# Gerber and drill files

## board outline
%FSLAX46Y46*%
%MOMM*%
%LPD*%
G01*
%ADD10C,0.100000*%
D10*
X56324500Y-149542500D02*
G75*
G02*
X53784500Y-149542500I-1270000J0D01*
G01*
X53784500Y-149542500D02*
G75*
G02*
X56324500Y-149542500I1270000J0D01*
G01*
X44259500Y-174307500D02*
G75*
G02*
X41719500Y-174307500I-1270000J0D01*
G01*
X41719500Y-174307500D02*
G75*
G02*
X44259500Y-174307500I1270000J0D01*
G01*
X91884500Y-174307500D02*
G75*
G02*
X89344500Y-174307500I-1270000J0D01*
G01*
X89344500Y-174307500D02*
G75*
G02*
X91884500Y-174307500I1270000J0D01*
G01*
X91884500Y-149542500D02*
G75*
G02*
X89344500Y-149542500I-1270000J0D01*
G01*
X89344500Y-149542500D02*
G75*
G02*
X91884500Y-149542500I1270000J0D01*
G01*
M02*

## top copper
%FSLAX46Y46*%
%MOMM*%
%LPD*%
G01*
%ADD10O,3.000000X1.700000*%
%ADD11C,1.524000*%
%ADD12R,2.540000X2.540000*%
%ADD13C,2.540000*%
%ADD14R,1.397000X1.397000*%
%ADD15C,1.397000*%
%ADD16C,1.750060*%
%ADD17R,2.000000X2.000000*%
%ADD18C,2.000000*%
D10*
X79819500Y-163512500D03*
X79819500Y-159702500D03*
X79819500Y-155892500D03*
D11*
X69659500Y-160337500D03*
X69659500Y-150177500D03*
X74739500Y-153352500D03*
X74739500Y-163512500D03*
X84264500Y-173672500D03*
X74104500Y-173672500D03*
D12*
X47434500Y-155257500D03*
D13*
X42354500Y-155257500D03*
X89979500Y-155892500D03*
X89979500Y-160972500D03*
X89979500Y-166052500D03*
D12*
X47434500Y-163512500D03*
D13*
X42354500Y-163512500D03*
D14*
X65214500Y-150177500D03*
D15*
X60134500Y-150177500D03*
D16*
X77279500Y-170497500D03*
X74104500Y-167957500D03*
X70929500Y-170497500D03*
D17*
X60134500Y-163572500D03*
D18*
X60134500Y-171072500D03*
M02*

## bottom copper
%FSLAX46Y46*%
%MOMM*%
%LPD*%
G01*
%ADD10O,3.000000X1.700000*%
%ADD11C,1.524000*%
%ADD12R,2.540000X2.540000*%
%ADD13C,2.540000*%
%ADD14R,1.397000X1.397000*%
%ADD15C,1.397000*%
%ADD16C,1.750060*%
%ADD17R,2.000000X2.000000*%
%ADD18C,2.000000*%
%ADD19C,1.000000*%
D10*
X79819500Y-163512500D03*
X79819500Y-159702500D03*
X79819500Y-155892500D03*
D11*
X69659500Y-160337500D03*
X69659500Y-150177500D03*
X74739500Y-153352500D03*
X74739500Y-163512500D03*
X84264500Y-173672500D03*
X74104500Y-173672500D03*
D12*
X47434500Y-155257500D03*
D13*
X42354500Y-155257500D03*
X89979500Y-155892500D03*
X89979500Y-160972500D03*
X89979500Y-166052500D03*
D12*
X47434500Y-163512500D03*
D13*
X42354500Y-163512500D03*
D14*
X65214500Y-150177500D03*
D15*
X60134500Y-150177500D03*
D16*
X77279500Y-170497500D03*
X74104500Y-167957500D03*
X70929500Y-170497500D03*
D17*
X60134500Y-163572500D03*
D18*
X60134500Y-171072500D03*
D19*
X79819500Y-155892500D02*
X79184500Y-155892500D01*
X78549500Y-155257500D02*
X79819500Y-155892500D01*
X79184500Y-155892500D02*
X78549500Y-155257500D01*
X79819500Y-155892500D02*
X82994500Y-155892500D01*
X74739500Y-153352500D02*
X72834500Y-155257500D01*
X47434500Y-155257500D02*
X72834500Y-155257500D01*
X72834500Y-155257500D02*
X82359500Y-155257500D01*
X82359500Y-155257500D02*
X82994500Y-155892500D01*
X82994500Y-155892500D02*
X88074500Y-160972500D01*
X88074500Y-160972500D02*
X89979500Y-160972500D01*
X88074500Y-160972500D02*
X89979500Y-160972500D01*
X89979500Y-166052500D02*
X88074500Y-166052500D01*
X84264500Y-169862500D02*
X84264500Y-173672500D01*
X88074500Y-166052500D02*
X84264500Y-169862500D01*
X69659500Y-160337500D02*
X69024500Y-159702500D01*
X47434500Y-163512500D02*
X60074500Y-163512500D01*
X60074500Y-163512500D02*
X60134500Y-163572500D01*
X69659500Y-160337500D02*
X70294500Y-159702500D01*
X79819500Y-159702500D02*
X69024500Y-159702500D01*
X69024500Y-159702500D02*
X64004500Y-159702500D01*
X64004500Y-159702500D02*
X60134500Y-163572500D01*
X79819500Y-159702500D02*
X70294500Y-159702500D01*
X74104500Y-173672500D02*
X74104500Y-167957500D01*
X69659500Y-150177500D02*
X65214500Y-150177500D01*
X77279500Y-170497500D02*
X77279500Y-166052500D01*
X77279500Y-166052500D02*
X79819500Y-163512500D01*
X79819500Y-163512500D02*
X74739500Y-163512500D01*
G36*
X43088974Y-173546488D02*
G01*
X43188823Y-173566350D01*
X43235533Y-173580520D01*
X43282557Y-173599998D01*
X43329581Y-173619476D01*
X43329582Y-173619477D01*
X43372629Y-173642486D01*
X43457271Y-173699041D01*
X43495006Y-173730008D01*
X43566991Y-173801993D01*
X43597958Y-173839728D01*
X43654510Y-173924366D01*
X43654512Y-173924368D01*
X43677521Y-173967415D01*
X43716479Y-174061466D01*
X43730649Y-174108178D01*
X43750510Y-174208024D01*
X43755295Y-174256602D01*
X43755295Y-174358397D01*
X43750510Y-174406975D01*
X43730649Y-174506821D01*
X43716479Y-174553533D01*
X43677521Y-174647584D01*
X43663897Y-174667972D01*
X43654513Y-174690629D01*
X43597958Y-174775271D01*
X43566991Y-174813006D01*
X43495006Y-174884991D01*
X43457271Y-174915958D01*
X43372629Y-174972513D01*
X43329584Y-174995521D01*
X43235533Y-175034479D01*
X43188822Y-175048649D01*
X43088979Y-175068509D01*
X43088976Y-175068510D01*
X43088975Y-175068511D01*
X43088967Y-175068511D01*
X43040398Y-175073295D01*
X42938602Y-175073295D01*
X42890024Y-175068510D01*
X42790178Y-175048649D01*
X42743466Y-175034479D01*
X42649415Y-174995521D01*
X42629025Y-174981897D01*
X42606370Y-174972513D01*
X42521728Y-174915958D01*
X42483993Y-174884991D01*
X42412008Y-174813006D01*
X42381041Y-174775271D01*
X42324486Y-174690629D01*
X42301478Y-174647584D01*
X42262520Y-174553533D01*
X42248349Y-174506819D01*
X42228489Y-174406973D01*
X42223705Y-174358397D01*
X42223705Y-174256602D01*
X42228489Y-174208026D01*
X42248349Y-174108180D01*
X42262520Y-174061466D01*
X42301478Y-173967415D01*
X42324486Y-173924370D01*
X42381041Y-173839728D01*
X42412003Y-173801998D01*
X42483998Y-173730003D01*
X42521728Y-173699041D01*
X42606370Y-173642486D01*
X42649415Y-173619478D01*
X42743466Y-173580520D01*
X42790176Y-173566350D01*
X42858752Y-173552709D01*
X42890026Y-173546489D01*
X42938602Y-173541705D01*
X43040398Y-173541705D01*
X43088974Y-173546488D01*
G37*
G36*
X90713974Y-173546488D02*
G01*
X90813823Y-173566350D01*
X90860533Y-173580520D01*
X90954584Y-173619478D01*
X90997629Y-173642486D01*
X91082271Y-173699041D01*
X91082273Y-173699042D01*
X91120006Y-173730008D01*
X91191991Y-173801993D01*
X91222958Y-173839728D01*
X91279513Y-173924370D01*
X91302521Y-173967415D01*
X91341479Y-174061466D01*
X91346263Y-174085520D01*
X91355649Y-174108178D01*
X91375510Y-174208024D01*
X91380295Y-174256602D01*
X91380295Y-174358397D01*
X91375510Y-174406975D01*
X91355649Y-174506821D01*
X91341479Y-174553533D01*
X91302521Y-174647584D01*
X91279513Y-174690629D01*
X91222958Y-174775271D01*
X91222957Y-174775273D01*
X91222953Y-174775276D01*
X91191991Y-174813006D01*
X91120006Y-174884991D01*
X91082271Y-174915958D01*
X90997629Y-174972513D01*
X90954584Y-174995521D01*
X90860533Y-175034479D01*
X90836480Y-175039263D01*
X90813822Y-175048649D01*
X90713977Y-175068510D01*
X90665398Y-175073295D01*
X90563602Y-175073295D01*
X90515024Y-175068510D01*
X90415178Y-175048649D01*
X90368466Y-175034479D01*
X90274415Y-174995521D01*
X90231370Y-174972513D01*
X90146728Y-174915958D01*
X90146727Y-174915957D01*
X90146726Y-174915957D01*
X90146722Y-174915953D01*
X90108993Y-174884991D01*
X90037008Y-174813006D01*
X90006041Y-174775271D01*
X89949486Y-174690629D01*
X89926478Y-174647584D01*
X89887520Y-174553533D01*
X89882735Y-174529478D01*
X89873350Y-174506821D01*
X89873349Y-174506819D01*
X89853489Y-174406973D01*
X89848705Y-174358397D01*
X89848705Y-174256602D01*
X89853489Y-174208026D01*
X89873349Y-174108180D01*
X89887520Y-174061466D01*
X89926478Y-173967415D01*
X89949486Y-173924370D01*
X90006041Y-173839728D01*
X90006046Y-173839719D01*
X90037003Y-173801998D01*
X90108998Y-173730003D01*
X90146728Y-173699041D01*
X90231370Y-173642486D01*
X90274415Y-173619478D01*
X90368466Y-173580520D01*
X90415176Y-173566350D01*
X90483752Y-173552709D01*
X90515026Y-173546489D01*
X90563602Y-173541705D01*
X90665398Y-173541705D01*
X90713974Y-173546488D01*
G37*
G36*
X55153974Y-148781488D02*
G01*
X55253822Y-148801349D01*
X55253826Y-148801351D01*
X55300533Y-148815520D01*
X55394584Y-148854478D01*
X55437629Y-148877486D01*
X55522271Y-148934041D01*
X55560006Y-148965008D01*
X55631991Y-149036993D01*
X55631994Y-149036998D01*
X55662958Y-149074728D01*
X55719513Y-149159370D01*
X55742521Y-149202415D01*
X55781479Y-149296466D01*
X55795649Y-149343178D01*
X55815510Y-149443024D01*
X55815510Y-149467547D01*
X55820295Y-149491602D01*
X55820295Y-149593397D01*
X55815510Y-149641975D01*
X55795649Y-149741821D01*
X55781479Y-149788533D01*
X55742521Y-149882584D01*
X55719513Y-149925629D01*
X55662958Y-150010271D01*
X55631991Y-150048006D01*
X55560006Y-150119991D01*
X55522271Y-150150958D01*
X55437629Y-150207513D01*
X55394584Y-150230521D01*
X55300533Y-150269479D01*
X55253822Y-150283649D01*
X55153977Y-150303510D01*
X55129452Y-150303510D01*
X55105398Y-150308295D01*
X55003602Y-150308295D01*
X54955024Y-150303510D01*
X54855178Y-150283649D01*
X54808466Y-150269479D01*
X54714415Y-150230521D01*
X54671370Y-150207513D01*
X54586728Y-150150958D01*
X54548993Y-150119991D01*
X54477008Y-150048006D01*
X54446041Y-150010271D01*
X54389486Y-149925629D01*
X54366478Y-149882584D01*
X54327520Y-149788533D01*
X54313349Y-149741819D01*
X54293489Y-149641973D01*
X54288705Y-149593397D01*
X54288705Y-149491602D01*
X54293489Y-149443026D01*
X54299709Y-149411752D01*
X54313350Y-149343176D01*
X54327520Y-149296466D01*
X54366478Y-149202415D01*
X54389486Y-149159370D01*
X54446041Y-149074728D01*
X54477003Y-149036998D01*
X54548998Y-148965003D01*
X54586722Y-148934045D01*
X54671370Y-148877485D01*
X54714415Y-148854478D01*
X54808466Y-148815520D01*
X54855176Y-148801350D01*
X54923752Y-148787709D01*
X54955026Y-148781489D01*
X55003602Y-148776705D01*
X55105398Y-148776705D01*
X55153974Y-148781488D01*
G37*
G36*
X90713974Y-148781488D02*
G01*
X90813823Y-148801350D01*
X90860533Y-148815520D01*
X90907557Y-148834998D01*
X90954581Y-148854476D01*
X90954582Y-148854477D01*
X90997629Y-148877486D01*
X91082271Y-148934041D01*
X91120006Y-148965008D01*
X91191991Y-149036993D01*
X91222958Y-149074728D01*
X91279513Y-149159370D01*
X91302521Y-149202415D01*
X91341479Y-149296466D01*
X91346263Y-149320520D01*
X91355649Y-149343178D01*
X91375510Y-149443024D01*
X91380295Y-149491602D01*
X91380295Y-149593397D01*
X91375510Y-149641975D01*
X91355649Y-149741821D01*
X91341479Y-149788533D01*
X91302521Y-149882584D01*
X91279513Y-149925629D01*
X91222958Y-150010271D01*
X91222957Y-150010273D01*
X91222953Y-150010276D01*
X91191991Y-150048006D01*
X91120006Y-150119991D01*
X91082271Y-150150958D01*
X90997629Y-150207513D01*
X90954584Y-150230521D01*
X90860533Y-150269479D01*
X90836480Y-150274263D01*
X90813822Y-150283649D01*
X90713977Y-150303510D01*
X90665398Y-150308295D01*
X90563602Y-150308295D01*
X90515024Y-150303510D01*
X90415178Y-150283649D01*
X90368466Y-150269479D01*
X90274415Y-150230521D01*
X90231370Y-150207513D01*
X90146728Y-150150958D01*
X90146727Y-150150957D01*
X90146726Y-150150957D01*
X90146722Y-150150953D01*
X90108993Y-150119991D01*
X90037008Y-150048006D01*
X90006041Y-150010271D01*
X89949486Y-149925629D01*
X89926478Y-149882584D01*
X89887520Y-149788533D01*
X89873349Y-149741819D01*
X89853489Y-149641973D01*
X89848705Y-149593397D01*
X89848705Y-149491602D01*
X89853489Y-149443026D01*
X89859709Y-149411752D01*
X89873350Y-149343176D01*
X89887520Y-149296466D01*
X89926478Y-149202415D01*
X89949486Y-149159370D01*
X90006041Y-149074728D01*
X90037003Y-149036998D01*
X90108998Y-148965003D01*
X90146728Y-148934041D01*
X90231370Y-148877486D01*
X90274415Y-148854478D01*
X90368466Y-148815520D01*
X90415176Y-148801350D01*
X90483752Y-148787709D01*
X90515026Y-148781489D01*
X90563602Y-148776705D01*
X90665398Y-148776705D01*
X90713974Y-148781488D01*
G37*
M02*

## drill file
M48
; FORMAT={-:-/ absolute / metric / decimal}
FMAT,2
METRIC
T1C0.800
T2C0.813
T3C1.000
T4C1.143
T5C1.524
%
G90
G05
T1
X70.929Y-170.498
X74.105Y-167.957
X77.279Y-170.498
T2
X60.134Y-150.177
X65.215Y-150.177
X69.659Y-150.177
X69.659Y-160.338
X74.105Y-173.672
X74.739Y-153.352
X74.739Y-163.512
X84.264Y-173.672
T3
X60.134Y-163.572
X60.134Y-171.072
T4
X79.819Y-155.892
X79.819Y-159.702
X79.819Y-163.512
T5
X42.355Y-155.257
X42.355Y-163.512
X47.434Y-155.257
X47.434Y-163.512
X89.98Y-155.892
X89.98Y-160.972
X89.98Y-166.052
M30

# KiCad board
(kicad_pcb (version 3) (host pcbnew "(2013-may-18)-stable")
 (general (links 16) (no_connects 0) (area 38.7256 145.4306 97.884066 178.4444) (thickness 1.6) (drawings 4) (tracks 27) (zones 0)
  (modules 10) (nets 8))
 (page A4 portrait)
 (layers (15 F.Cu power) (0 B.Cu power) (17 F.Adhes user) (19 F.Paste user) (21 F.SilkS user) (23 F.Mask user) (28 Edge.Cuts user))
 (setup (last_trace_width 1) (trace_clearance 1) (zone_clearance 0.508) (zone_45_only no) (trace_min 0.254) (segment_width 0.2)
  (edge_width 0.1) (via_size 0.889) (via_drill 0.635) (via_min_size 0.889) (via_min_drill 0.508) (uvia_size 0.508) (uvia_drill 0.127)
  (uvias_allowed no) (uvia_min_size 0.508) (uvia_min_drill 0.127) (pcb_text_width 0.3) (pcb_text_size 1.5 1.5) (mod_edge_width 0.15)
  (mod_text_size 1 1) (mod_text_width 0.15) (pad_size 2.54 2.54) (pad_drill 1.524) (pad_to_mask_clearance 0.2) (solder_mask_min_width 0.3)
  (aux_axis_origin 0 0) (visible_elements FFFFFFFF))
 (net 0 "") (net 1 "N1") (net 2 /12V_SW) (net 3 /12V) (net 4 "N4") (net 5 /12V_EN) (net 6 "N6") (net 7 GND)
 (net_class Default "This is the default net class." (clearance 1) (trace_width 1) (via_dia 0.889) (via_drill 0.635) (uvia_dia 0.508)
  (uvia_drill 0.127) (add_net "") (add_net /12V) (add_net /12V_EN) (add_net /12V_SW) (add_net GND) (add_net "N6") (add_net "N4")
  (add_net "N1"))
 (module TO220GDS (layer F.Cu) (at 79.8195 159.7025 180)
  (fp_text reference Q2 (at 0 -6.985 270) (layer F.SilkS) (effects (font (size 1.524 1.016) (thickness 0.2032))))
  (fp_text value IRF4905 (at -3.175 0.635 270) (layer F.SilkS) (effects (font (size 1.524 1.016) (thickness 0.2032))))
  (pad G thru_hole oval (at 0 -3.81 180) (size 3 1.7) (drill 1.143) (layers *.Cu *.Mask F.SilkS) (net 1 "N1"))
  (pad D thru_hole oval (at 0 0 180) (size 3 1.7) (drill 1.143) (layers *.Cu *.Mask F.SilkS) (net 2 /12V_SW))
  (pad S thru_hole oval (at 0 3.81 180) (size 3 1.7) (drill 1.143) (layers *.Cu *.Mask F.SilkS) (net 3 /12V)))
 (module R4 (layer F.Cu) (at 69.6595 155.2575 90) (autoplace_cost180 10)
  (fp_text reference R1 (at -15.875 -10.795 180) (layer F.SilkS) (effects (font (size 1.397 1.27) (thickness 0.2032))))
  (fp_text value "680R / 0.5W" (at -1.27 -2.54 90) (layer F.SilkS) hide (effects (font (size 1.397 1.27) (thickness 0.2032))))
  (pad 1 thru_hole circle (at -5.08 0 90) (size 1.524 1.524) (drill 0.8128) (layers *.Cu *.Mask F.SilkS) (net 2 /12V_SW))
  (pad 2 thru_hole circle (at 5.08 0 90) (size 1.524 1.524) (drill 0.8128) (layers *.Cu *.Mask F.SilkS) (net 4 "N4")))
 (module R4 (layer F.Cu) (at 74.7395 158.4325 270) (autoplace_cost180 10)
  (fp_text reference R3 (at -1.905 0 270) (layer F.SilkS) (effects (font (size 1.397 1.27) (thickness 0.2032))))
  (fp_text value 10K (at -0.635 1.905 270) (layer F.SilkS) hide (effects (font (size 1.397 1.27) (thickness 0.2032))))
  (pad 1 thru_hole circle (at -5.08 0 270) (size 1.524 1.524) (drill 0.8128) (layers *.Cu *.Mask F.SilkS) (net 3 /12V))
  (pad 2 thru_hole circle (at 5.08 0 270) (size 1.524 1.524) (drill 0.8128) (layers *.Cu *.Mask F.SilkS) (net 1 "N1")))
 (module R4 (layer F.Cu) (at 79.1845 173.6725 180) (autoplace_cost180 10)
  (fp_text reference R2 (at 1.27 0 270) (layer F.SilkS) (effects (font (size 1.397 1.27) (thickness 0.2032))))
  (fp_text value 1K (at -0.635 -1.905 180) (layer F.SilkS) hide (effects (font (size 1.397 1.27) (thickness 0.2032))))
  (pad 1 thru_hole circle (at -5.08 0 180) (size 1.524 1.524) (drill 0.8128) (layers *.Cu *.Mask F.SilkS) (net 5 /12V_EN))
  (pad 2 thru_hole circle (at 5.08 0 180) (size 1.524 1.524) (drill 0.8128) (layers *.Cu *.Mask F.SilkS) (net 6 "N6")))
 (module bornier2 (layer F.Cu) (at 44.8945 155.2575 180)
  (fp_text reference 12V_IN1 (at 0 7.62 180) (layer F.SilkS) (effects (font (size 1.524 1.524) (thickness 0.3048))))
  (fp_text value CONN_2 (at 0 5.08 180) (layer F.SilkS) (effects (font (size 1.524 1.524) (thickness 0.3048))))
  (pad 1 thru_hole rect (at -2.54 0 180) (size 2.54 2.54) (drill 1.524) (layers *.Cu *.Mask F.SilkS) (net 3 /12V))
  (pad 2 thru_hole circle (at 2.54 0 180) (size 2.54 2.54) (drill 1.524) (layers *.Cu *.Mask F.SilkS) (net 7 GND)))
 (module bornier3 (layer F.Cu) (at 89.9795 160.9725 270)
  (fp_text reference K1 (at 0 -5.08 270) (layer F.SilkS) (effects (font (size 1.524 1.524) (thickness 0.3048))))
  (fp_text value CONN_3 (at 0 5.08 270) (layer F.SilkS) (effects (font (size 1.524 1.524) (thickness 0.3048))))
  (pad 1 thru_hole circle (at -5.08 0 270) (size 2.54 2.54) (drill 1.524) (layers *.Cu *.Mask F.SilkS) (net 7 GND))
  (pad 2 thru_hole circle (at 0 0 270) (size 2.54 2.54) (drill 1.524) (layers *.Cu *.Mask F.SilkS) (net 3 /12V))
  (pad 3 thru_hole circle (at 5.08 0 270) (size 2.54 2.54) (drill 1.524) (layers *.Cu *.Mask F.SilkS) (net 5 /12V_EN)))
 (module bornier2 (layer F.Cu) (at 44.8945 163.5125 180)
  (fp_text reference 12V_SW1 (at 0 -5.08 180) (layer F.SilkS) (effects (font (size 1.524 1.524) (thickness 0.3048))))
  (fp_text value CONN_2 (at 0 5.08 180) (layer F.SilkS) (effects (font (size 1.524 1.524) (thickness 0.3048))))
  (pad 1 thru_hole rect (at -2.54 0 180) (size 2.54 2.54) (drill 1.524) (layers *.Cu *.Mask F.SilkS) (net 2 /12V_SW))
  (pad 2 thru_hole circle (at 2.54 0 180) (size 2.54 2.54) (drill 1.524) (layers *.Cu *.Mask F.SilkS) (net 7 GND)))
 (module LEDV (layer F.Cu) (at 62.6745 150.1775 180)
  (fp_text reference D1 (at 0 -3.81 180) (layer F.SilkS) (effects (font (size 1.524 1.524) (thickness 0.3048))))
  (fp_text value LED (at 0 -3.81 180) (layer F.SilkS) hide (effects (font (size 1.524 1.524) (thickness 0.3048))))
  (pad 1 thru_hole rect (at -2.54 0 180) (size 1.397 1.397) (drill 0.8128) (layers *.Cu *.Mask F.SilkS) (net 4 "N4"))
  (pad 2 thru_hole circle (at 2.54 0 180) (size 1.397 1.397) (drill 0.8128) (layers *.Cu *.Mask F.SilkS) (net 7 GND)))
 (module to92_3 (layer F.Cu) (at 74.1045 169.8625)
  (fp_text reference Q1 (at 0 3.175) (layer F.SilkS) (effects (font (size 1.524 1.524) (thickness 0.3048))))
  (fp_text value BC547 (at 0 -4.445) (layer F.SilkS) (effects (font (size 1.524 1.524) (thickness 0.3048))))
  (pad 1 thru_hole circle (at 3.175 0.635) (size 1.75006 1.75006) (drill 0.8001) (layers *.Cu *.Mask F.SilkS) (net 1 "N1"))
  (pad 2 thru_hole circle (at 0 -1.905) (size 1.75006 1.75006) (drill 0.8001) (layers *.Cu *.Mask F.SilkS) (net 6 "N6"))
  (pad 3 thru_hole circle (at -3.175 0.635) (size 1.75006 1.75006) (drill 0.8001) (layers *.Cu *.Mask F.SilkS) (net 7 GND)))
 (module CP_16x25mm (layer F.Cu) (at 60.1345 167.3225 180)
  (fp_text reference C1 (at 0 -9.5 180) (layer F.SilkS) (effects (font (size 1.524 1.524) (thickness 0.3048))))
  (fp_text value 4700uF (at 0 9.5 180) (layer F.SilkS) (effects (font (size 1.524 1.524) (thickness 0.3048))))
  (pad 1 thru_hole rect (at 0 3.75 180) (size 2 2) (drill 1) (layers *.Cu *.Mask F.SilkS) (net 2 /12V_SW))
  (pad 2 thru_hole circle (at 0 -3.75 180) (size 2 2) (drill 1) (layers *.Cu *.Mask F.SilkS) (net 7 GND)))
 (gr_circle (center 55.0545 149.5425) (end 55.0545 150.8125) (layer Edge.Cuts) (width 0.1))
 (gr_circle (center 42.9895 174.3075) (end 42.9895 175.5775) (layer Edge.Cuts) (width 0.1))
 (gr_circle (center 90.6145 174.3075) (end 91.8845 174.3075) (layer Edge.Cuts) (width 0.1))
 (gr_circle (center 90.6145 149.5425) (end 89.3445 149.5425) (layer Edge.Cuts) (width 0.1))
 (segment (start 79.8195 155.8925) (end 79.1845 155.8925) (width 1) (layer B.Cu) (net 3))
 (segment (start 78.5495 155.2575) (end 79.8195 155.8925) (width 1) (layer B.Cu) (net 3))
 (segment (start 79.1845 155.8925) (end 78.5495 155.2575) (width 1) (layer B.Cu) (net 3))
 (segment (start 79.8195 155.8925) (end 82.9945 155.8925) (width 1) (layer B.Cu) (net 3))
 (segment (start 74.7395 153.3525) (end 72.8345 155.2575) (width 1) (layer B.Cu) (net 3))
 (segment (start 47.4345 155.2575) (end 72.8345 155.2575) (width 1) (layer B.Cu) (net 3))
 (segment (start 72.8345 155.2575) (end 82.3595 155.2575) (width 1) (layer B.Cu) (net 3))
 (segment (start 82.3595 155.2575) (end 82.9945 155.8925) (width 1) (layer B.Cu) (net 3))
 (segment (start 82.9945 155.8925) (end 88.0745 160.9725) (width 1) (layer B.Cu) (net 3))
 (segment (start 88.0745 160.9725) (end 89.9795 160.9725) (width 1) (layer B.Cu) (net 3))
 (segment (start 88.0745 160.9725) (end 89.9795 160.9725) (width 1) (layer B.Cu) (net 3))
 (segment (start 89.9795 166.0525) (end 88.0745 166.0525) (width 1) (layer B.Cu) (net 5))
 (segment (start 84.2645 169.8625) (end 84.2645 173.6725) (width 1) (layer B.Cu) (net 5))
 (segment (start 88.0745 166.0525) (end 84.2645 169.8625) (width 1) (layer B.Cu) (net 5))
 (segment (start 69.6595 160.3375) (end 69.0245 159.7025) (width 1) (layer B.Cu) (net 2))
 (segment (start 47.4345 163.5125) (end 60.0745 163.5125) (width 1) (layer B.Cu) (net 2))
 (segment (start 60.0745 163.5125) (end 60.1345 163.5725) (width 1) (layer B.Cu) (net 2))
 (segment (start 69.6595 160.3375) (end 70.2945 159.7025) (width 1) (layer B.Cu) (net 2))
 (segment (start 79.8195 159.7025) (end 69.0245 159.7025) (width 1) (layer B.Cu) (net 2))
 (segment (start 69.0245 159.7025) (end 64.0045 159.7025) (width 1) (layer B.Cu) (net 2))
 (segment (start 64.0045 159.7025) (end 60.1345 163.5725) (width 1) (layer B.Cu) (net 2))
 (segment (start 79.8195 159.7025) (end 70.2945 159.7025) (width 1) (layer B.Cu) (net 2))
 (segment (start 74.1045 173.6725) (end 74.1045 167.9575) (width 1) (layer B.Cu) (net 6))
 (segment (start 69.6595 150.1775) (end 65.2145 150.1775) (width 1) (layer B.Cu) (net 4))
 (segment (start 77.2795 170.4975) (end 77.2795 166.0525) (width 1) (layer B.Cu) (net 1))
 (segment (start 77.2795 166.0525) (end 79.8195 163.5125) (width 1) (layer B.Cu) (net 1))
 (segment (start 79.8195 163.5125) (end 74.7395 163.5125) (width 1) (layer B.Cu) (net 1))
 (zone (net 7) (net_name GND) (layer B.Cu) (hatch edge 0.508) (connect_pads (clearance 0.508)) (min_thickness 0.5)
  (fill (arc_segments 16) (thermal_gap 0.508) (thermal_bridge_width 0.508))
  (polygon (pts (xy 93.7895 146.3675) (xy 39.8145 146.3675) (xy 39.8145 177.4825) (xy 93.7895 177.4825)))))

